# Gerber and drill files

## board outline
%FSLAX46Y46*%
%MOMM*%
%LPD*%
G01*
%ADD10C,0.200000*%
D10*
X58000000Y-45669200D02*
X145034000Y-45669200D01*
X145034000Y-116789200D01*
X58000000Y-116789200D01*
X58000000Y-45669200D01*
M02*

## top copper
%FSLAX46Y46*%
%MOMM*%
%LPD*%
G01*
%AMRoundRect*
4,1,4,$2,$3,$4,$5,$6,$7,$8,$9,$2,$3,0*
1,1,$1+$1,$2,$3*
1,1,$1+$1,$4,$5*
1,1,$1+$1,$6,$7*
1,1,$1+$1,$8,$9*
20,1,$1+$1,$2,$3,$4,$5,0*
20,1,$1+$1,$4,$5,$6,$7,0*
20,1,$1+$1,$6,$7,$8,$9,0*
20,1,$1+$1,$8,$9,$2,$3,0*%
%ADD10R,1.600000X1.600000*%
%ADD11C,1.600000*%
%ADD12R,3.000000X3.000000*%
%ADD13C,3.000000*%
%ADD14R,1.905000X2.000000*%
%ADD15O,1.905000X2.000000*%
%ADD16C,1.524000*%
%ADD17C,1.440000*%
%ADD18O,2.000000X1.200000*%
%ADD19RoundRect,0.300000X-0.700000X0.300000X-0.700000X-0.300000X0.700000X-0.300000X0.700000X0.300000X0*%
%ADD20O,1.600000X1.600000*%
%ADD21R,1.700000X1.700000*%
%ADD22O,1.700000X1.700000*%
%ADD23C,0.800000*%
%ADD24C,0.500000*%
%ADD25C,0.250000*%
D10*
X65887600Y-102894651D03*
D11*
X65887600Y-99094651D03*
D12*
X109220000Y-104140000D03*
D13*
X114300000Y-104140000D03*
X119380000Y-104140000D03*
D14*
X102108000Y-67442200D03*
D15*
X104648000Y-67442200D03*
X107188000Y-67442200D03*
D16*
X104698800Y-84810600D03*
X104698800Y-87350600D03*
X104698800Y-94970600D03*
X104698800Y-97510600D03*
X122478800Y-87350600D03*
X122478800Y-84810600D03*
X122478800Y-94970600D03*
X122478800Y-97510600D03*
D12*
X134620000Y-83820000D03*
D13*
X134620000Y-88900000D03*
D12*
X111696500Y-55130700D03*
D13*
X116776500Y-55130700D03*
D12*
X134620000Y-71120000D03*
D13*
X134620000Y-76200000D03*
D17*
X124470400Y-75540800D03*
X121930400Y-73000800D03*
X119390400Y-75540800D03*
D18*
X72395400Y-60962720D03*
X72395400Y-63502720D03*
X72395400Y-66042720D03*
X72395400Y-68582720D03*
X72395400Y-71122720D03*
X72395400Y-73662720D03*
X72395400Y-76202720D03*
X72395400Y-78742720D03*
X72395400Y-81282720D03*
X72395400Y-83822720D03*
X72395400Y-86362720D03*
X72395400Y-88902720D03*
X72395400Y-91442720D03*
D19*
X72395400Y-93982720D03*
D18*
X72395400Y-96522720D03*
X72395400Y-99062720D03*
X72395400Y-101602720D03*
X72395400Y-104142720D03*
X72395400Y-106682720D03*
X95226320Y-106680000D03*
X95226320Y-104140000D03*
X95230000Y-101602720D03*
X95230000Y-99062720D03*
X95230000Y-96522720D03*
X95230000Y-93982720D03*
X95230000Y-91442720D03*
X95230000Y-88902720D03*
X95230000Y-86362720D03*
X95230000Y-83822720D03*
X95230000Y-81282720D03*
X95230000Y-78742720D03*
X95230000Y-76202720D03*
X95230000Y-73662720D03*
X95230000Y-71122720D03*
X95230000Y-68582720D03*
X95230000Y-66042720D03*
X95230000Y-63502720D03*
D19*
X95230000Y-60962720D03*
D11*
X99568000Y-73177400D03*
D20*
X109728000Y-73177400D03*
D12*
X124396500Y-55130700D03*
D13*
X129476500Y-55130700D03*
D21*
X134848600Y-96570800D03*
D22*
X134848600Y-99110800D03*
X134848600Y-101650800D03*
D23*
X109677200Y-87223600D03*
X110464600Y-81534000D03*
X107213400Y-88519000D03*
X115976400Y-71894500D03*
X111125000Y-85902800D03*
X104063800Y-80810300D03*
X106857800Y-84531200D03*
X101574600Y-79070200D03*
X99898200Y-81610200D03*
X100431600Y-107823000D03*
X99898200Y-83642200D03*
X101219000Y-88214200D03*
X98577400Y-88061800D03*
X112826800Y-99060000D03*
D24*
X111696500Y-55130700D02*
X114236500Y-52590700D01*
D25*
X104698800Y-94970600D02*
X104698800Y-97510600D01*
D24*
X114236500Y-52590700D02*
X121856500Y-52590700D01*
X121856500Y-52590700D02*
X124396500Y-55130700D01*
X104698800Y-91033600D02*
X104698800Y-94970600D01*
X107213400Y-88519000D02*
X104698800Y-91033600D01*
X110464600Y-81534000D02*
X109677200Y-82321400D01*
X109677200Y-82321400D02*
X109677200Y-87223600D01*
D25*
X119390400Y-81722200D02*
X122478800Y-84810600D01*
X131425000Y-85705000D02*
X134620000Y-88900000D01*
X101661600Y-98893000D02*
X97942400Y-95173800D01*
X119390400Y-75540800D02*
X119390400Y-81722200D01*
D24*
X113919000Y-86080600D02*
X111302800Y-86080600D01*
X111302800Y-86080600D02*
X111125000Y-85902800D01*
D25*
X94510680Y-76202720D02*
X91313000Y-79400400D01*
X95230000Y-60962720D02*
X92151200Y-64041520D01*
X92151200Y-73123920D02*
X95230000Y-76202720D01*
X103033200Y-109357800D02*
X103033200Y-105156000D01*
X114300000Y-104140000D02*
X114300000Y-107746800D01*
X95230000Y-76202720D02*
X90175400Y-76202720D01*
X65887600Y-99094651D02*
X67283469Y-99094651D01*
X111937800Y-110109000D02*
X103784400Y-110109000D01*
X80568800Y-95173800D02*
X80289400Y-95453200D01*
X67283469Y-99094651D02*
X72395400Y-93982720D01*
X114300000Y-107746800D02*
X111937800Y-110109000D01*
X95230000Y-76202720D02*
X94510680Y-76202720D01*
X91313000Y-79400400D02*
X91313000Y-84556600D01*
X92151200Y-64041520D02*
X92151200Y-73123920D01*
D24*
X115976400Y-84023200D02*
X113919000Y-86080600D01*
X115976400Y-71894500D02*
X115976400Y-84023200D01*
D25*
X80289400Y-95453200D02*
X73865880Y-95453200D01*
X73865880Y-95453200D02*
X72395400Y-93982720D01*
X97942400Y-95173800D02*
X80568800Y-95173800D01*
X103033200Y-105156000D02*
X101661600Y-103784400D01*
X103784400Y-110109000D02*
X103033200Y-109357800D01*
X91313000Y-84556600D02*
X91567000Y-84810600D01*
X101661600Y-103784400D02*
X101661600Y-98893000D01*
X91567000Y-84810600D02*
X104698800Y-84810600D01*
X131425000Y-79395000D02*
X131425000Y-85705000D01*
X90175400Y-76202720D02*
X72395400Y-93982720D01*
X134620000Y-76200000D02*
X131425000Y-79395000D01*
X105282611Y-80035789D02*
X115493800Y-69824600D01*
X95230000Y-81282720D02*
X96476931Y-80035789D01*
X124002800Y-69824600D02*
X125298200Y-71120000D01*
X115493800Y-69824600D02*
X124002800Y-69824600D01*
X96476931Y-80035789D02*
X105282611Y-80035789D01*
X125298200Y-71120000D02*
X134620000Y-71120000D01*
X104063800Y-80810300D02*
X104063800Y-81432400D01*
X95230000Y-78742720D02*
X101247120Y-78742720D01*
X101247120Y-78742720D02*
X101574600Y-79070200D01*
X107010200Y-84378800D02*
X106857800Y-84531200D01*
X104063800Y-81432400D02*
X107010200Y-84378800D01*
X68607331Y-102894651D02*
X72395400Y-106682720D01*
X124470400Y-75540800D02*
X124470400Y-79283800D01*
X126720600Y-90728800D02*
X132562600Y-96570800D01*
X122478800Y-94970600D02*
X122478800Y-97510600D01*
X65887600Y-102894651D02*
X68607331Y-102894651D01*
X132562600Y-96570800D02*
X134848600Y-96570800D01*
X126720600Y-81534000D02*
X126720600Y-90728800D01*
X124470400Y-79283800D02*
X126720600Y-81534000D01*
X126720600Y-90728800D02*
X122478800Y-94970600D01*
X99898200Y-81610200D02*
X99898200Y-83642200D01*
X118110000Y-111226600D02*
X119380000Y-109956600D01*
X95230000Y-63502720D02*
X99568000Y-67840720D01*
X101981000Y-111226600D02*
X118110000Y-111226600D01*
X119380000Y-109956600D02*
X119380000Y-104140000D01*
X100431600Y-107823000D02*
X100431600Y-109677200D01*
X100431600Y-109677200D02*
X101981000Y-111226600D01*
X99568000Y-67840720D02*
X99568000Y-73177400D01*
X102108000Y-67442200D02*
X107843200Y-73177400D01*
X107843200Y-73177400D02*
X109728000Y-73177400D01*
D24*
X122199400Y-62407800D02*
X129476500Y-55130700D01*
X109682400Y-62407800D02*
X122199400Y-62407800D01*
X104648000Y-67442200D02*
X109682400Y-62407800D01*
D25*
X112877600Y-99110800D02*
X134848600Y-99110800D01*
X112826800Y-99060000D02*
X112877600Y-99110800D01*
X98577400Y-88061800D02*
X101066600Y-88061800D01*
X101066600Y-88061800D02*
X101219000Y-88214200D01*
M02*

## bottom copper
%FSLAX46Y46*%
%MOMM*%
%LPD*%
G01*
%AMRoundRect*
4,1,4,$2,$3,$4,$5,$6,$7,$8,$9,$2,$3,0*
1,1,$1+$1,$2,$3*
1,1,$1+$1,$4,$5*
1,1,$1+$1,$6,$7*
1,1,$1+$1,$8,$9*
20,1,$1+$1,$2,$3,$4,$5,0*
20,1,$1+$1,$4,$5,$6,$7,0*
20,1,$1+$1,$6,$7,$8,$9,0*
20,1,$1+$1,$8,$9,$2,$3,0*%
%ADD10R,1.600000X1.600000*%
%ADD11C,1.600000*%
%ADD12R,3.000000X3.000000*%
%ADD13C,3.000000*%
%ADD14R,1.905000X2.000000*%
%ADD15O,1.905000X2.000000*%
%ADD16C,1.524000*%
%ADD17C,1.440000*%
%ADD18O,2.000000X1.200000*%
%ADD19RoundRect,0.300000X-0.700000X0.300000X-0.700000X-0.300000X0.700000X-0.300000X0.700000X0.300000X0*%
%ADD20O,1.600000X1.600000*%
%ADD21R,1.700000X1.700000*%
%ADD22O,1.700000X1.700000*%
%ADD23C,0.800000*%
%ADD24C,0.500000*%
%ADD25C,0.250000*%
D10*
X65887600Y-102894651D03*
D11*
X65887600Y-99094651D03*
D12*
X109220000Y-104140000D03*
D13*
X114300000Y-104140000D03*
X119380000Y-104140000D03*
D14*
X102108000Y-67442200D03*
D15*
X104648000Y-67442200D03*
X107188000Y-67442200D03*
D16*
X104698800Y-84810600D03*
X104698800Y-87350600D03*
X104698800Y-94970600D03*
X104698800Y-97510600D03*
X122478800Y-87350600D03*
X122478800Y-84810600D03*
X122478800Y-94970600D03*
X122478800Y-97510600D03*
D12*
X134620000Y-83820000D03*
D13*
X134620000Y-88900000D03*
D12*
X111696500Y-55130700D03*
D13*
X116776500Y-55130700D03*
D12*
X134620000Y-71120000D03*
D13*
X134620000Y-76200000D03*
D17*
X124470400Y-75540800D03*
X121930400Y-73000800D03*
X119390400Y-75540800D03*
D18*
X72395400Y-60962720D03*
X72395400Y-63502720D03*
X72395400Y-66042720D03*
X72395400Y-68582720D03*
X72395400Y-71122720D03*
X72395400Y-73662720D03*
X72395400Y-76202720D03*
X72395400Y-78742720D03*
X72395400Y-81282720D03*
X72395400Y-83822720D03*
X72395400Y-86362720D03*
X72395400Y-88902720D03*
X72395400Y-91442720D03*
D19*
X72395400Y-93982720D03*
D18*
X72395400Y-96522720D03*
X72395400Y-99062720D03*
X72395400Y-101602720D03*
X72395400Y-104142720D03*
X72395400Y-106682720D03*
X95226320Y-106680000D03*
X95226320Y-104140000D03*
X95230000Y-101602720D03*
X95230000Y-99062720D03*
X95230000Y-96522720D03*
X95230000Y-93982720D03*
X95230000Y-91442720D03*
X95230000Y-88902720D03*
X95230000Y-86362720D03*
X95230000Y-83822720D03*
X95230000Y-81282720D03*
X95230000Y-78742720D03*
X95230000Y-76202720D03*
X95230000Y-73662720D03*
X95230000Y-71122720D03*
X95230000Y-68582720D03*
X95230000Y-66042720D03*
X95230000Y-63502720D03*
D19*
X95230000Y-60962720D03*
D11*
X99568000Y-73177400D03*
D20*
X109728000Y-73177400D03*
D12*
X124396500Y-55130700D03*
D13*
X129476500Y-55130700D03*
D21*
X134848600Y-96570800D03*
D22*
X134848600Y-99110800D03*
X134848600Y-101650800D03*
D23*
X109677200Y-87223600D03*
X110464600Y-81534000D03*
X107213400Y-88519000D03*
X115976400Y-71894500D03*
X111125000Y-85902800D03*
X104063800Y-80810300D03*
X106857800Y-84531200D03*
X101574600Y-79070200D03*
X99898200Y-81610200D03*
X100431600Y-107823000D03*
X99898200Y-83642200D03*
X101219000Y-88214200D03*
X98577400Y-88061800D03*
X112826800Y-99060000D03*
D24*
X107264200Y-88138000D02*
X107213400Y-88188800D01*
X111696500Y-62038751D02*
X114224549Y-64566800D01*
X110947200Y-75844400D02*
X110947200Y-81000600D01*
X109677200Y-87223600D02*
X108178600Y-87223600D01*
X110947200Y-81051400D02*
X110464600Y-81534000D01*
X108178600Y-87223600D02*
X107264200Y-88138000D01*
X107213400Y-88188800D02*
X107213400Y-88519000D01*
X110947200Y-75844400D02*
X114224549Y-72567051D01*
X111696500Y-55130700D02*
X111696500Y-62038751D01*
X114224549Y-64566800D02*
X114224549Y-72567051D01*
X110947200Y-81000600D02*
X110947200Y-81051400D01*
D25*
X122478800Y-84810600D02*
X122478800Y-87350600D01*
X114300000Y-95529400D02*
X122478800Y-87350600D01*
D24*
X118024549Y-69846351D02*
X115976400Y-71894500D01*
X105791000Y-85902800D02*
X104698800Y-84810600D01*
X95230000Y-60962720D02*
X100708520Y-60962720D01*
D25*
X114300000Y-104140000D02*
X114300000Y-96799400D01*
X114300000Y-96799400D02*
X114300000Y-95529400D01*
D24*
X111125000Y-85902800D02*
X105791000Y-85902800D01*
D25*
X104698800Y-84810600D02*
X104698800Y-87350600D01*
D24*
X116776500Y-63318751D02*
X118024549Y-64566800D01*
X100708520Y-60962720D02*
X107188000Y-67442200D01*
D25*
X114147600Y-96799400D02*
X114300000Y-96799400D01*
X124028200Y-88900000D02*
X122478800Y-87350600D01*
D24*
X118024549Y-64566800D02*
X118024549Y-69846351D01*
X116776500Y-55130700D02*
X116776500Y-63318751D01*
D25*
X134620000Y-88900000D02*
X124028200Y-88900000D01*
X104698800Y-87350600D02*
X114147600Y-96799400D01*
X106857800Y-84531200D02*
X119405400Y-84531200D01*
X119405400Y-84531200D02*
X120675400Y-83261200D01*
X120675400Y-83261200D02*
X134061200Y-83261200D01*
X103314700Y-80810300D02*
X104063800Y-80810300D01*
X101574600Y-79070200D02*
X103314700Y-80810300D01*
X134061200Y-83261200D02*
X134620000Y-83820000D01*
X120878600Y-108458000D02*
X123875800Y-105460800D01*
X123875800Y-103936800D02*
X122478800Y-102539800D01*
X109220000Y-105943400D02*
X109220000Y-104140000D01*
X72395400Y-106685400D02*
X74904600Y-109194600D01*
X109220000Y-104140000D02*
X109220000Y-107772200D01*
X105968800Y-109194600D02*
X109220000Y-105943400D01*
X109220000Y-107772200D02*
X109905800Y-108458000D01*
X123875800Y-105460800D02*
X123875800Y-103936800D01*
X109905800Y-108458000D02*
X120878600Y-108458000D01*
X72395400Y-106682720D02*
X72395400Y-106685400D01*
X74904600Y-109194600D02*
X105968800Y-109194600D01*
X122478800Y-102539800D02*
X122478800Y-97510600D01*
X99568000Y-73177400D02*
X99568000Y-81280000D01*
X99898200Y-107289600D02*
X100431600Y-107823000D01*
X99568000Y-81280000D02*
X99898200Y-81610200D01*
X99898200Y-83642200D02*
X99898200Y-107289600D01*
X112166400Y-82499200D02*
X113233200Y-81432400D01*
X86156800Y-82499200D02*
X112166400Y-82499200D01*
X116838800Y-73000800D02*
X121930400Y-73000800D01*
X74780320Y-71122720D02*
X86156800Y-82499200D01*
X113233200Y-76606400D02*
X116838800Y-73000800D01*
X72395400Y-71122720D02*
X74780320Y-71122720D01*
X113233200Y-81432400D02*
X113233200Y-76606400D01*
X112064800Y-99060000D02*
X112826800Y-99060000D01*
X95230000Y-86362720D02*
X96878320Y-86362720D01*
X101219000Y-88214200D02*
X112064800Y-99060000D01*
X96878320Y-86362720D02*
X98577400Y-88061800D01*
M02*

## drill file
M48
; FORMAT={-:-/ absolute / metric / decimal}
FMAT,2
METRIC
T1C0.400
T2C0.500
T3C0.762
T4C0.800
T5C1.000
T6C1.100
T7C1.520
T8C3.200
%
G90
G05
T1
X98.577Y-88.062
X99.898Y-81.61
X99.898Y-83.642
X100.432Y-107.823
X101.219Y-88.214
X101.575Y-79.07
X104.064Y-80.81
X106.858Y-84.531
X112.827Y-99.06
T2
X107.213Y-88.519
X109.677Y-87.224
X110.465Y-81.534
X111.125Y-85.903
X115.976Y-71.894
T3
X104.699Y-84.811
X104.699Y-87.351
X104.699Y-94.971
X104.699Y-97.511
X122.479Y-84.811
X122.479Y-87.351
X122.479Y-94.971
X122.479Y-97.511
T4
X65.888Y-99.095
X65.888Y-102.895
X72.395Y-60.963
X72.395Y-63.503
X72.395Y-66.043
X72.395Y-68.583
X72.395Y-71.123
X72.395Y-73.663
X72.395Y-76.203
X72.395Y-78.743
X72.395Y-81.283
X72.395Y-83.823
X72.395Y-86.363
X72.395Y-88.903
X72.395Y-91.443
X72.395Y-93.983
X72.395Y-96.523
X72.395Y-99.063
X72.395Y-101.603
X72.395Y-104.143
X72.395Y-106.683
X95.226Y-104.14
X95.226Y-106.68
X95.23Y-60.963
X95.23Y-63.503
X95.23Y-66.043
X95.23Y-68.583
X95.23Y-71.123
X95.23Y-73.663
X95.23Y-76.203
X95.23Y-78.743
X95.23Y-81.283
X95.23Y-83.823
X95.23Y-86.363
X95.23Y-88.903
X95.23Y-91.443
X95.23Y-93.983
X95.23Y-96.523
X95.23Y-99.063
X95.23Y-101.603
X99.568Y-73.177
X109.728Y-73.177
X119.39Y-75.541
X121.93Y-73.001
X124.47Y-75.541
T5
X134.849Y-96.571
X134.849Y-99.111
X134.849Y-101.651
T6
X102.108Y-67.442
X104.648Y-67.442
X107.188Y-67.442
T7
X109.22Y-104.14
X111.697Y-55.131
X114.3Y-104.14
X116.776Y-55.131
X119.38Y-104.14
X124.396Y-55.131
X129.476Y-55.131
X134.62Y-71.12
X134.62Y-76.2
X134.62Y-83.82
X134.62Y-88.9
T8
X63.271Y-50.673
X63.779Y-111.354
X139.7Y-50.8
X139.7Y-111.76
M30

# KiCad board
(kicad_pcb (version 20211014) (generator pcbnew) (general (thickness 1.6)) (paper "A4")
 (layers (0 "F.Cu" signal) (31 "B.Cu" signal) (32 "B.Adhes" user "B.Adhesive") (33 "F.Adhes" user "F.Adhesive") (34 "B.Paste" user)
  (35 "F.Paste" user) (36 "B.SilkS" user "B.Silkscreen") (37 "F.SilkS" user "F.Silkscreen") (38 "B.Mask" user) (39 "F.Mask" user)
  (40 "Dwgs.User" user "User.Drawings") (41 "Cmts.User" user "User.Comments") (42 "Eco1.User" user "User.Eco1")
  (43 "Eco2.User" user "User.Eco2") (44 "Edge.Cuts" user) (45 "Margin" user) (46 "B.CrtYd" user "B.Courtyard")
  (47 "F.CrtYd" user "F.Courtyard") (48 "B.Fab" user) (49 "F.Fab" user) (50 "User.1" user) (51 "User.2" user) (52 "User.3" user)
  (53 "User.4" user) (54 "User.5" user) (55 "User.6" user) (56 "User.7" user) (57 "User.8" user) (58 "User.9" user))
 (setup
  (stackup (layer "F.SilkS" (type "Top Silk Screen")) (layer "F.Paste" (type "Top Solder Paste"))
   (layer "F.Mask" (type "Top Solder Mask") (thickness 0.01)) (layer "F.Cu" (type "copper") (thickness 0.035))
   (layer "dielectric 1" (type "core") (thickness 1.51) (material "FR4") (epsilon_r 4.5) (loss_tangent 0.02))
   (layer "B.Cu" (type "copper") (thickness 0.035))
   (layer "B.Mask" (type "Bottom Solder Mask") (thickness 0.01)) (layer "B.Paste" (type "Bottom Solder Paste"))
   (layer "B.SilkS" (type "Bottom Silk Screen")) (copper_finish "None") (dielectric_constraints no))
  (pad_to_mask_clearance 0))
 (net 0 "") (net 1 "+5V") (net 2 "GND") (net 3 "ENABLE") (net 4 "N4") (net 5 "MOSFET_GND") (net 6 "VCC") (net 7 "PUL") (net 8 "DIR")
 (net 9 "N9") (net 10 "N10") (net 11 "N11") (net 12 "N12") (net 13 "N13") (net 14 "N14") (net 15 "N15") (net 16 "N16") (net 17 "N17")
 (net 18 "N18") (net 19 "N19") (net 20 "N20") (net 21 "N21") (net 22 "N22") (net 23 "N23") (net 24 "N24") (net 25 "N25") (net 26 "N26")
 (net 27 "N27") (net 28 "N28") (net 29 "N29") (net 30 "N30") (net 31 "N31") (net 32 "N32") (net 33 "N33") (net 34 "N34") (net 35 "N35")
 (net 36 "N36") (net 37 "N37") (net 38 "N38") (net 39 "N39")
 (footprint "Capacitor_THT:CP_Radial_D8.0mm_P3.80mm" (layer "F.Cu") (at 65.8876 102.894651 90)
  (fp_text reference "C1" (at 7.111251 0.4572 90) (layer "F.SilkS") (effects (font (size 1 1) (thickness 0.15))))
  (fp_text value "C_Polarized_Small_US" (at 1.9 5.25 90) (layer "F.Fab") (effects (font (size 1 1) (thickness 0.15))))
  (pad "1" thru_hole rect (at 0 0 90) (size 1.6 1.6) (drill 0.8) (layers *.Cu *.Mask) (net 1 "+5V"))
  (pad "2" thru_hole circle (at 3.8 0 90) (size 1.6 1.6) (drill 0.8) (layers *.Cu *.Mask) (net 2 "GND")))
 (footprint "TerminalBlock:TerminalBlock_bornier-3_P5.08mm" (layer "F.Cu") (at 109.22 104.14)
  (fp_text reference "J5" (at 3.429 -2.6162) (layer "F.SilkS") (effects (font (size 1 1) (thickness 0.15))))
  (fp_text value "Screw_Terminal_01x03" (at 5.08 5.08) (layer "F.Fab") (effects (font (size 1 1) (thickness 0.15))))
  (pad "1" thru_hole rect (at 0 0) (size 3 3) (drill 1.52) (layers *.Cu *.Mask) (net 1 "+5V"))
  (pad "2" thru_hole circle (at 5.08 0) (size 3 3) (drill 1.52) (layers *.Cu *.Mask) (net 2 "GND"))
  (pad "3" thru_hole circle (at 10.16 0) (size 3 3) (drill 1.52) (layers *.Cu *.Mask) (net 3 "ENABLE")))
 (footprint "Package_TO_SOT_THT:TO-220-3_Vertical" (layer "F.Cu") (at 102.108 67.4422)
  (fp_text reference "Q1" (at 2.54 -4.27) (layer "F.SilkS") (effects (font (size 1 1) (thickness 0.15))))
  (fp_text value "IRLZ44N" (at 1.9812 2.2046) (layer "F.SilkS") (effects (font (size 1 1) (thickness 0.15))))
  (pad "1" thru_hole rect (at 0 0) (size 1.905 2) (drill 1.1) (layers *.Cu *.Mask) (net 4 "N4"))
  (pad "2" thru_hole oval (at 2.54 0) (size 1.905 2) (drill 1.1) (layers *.Cu *.Mask) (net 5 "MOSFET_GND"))
  (pad "3" thru_hole oval (at 5.08 0) (size 1.905 2) (drill 1.1) (layers *.Cu *.Mask) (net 2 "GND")))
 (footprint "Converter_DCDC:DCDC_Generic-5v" (layer "F.Cu") (at 114.8588 92.4306)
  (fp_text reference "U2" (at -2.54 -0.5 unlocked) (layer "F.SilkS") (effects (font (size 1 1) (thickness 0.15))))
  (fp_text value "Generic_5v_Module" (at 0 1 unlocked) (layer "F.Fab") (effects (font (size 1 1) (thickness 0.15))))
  (pad "1" thru_hole circle (at -10.16 -7.62) (size 1.524 1.524) (drill 0.762) (layers *.Cu *.Mask) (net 2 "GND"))
  (pad "1" thru_hole circle (at -10.16 -5.08) (size 1.524 1.524) (drill 0.762) (layers *.Cu *.Mask) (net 2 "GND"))
  (pad "2" thru_hole circle (at -10.16 2.54) (size 1.524 1.524) (drill 0.762) (layers *.Cu *.Mask) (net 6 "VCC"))
  (pad "2" thru_hole circle (at -10.16 5.08) (size 1.524 1.524) (drill 0.762) (layers *.Cu *.Mask) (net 6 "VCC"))
  (pad "3" thru_hole circle (at 7.62 -5.08) (size 1.524 1.524) (drill 0.762) (layers *.Cu *.Mask) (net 2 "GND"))
  (pad "3" thru_hole circle (at 7.62 -7.62) (size 1.524 1.524) (drill 0.762) (layers *.Cu *.Mask) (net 2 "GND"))
  (pad "4" thru_hole circle (at 7.62 2.54) (size 1.524 1.524) (drill 0.762) (layers *.Cu *.Mask) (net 1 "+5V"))
  (pad "4" thru_hole circle (at 7.62 5.08) (size 1.524 1.524) (drill 0.762) (layers *.Cu *.Mask) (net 1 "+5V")))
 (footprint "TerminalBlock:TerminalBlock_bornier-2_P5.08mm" (layer "F.Cu") (at 134.62 83.82 -90)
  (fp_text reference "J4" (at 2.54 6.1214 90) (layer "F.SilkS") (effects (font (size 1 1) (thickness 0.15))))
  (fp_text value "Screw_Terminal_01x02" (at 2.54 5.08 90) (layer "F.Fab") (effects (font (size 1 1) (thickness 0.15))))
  (pad "1" thru_hole rect (at 0 0 270) (size 3 3) (drill 1.52) (layers *.Cu *.Mask) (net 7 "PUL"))
  (pad "2" thru_hole circle (at 5.08 0 270) (size 3 3) (drill 1.52) (layers *.Cu *.Mask) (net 2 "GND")))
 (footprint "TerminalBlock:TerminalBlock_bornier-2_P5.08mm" (layer "F.Cu") (at 111.6965 55.1307)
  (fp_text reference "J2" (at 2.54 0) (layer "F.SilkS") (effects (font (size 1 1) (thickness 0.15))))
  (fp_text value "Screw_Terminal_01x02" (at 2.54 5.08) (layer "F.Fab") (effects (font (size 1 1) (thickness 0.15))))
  (pad "1" thru_hole rect (at 0 0) (size 3 3) (drill 1.52) (layers *.Cu *.Mask) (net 6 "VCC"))
  (pad "2" thru_hole circle (at 5.08 0) (size 3 3) (drill 1.52) (layers *.Cu *.Mask) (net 2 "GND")))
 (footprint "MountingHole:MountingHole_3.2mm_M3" (layer "F.Cu") (at 63.2714 50.673)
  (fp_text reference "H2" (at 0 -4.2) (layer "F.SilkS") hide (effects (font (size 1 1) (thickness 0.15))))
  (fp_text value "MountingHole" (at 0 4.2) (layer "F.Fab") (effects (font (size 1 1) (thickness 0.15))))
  (pad "" np_thru_hole circle (at 0 0) (size 3.2 3.2) (drill 3.2) (layers *.Cu *.Mask)))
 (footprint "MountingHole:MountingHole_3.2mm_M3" (layer "F.Cu") (at 139.7 111.76)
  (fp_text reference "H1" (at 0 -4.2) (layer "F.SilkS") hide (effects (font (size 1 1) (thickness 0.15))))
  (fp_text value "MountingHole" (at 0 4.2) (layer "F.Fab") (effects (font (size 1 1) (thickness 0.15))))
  (pad "" np_thru_hole circle (at 0 0) (size 3.2 3.2) (drill 3.2) (layers *.Cu *.Mask)))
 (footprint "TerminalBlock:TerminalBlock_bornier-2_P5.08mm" (layer "F.Cu") (at 134.62 71.12 -90)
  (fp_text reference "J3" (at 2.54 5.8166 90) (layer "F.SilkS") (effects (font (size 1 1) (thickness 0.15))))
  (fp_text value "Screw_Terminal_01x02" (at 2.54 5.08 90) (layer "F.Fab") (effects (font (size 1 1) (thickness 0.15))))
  (pad "1" thru_hole rect (at 0 0 270) (size 3 3) (drill 1.52) (layers *.Cu *.Mask) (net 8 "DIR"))
  (pad "2" thru_hole circle (at 5.08 0 270) (size 3 3) (drill 1.52) (layers *.Cu *.Mask) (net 2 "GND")))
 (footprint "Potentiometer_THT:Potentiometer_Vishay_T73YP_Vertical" (layer "F.Cu") (at 124.4704 75.5408 90)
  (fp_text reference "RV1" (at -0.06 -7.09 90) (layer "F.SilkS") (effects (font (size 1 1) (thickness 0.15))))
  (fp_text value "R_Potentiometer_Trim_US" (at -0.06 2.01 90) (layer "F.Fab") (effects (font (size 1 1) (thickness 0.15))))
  (pad "1" thru_hole circle (at 0 0 90) (size 1.44 1.44) (drill 0.8) (layers *.Cu *.Mask) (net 1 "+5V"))
  (pad "2" thru_hole circle (at 2.54 -2.54 90) (size 1.44 1.44) (drill 0.8) (layers *.Cu *.Mask) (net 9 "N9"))
  (pad "3" thru_hole circle (at 0 -5.08 90) (size 1.44 1.44) (drill 0.8) (layers *.Cu *.Mask) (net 2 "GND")))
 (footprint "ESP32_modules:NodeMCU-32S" (layer "F.Cu") (at 71.12 60.96)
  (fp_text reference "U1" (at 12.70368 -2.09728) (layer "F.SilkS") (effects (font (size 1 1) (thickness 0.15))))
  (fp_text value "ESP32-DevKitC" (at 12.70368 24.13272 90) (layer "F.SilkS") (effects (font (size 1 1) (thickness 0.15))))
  (pad "1" thru_hole oval (at 1.2754 0.00272 270) (size 1.2 2) (drill 0.8) (layers *.Cu *.Mask) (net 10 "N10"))
  (pad "2" thru_hole oval (at 1.2754 2.54272 270) (size 1.2 2) (drill 0.8) (layers *.Cu *.Mask) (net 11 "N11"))
  (pad "3" thru_hole oval (at 1.2754 5.08272 270) (size 1.2 2) (drill 0.8) (layers *.Cu *.Mask) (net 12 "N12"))
  (pad "4" thru_hole oval (at 1.2754 7.62272 270) (size 1.2 2) (drill 0.8) (layers *.Cu *.Mask) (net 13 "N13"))
  (pad "5" thru_hole oval (at 1.2754 10.16272 270) (size 1.2 2) (drill 0.8) (layers *.Cu *.Mask) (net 9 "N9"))
  (pad "6" thru_hole oval (at 1.2754 12.70272 270) (size 1.2 2) (drill 0.8) (layers *.Cu *.Mask) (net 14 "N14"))
  (pad "7" thru_hole oval (at 1.2754 15.24272 270) (size 1.2 2) (drill 0.8) (layers *.Cu *.Mask) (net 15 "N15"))
  (pad "8" thru_hole oval (at 1.2754 17.78272 270) (size 1.2 2) (drill 0.8) (layers *.Cu *.Mask) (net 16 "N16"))
  (pad "9" thru_hole oval (at 1.2754 20.32272 270) (size 1.2 2) (drill 0.8) (layers *.Cu *.Mask) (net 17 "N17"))
  (pad "10" thru_hole oval (at 1.2754 22.86272 270) (size 1.2 2) (drill 0.8) (layers *.Cu *.Mask) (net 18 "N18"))
  (pad "11" thru_hole oval (at 1.2754 25.40272 270) (size 1.2 2) (drill 0.8) (layers *.Cu *.Mask) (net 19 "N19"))
  (pad "12" thru_hole oval (at 1.2754 27.94272 270) (size 1.2 2) (drill 0.8) (layers *.Cu *.Mask) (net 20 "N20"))
  (pad "13" thru_hole oval (at 1.2754 30.48272 270) (size 1.2 2) (drill 0.8) (layers *.Cu *.Mask) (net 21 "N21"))
  (pad "14" thru_hole roundrect (at 1.2754 33.02272 270) (size 1.2 2) (drill 0.8) (layers *.Cu *.Mask) (roundrect_rratio 0.25) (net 2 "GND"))
  (pad "15" thru_hole oval (at 1.2754 35.56272 270) (size 1.2 2) (drill 0.8) (layers *.Cu *.Mask) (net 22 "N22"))
  (pad "16" thru_hole oval (at 1.2754 38.10272 270) (size 1.2 2) (drill 0.8) (layers *.Cu *.Mask) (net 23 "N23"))
  (pad "17" thru_hole oval (at 1.2754 40.64272 270) (size 1.2 2) (drill 0.8) (layers *.Cu *.Mask) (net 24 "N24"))
  (pad "18" thru_hole oval (at 1.2754 43.18272 270) (size 1.2 2) (drill 0.8) (layers *.Cu *.Mask) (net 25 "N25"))
  (pad "19" thru_hole oval (at 1.2754 45.72272 270) (size 1.2 2) (drill 0.8) (layers *.Cu *.Mask) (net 1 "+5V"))
  (pad "20" thru_hole oval (at 24.10632 45.72 270) (size 1.2 2) (drill 0.8) (layers *.Cu *.Mask) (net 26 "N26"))
  (pad "21" thru_hole oval (at 24.10632 43.18 270) (size 1.2 2) (drill 0.8) (layers *.Cu *.Mask) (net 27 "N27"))
  (pad "22" thru_hole oval (at 24.11 40.64272 270) (size 1.2 2) (drill 0.8) (layers *.Cu *.Mask) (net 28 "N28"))
  (pad "23" thru_hole oval (at 24.11 38.10272 270) (size 1.2 2) (drill 0.8) (layers *.Cu *.Mask) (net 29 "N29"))
  (pad "24" thru_hole oval (at 24.11 35.56272 270) (size 1.2 2) (drill 0.8) (layers *.Cu *.Mask) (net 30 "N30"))
  (pad "25" thru_hole oval (at 24.11 33.02272 270) (size 1.2 2) (drill 0.8) (layers *.Cu *.Mask) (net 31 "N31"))
  (pad "26" thru_hole oval (at 24.11 30.48272 270) (size 1.2 2) (drill 0.8) (layers *.Cu *.Mask) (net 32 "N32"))
  (pad "27" thru_hole oval (at 24.11 27.94272 270) (size 1.2 2) (drill 0.8) (layers *.Cu *.Mask) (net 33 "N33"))
  (pad "28" thru_hole oval (at 24.11 25.40272 270) (size 1.2 2) (drill 0.8) (layers *.Cu *.Mask) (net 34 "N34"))
  (pad "29" thru_hole oval (at 24.11 22.86272 270) (size 1.2 2) (drill 0.8) (layers *.Cu *.Mask) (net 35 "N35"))
  (pad "30" thru_hole oval (at 24.11 20.32272 270) (size 1.2 2) (drill 0.8) (layers *.Cu *.Mask) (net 8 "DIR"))
  (pad "31" thru_hole oval (at 24.11 17.78272 270) (size 1.2 2) (drill 0.8) (layers *.Cu *.Mask) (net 7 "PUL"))
  (pad "32" thru_hole oval (at 24.11 15.24272 270) (size 1.2 2) (drill 0.8) (layers *.Cu *.Mask) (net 2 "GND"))
  (pad "33" thru_hole oval (at 24.11 12.70272 270) (size 1.2 2) (drill 0.8) (layers *.Cu *.Mask) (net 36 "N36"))
  (pad "34" thru_hole oval (at 24.11 10.16272 270) (size 1.2 2) (drill 0.8) (layers *.Cu *.Mask) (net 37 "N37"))
  (pad "35" thru_hole oval (at 24.11 7.62272 270) (size 1.2 2) (drill 0.8) (layers *.Cu *.Mask) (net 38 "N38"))
  (pad "36" thru_hole oval (at 24.11 5.08272 270) (size 1.2 2) (drill 0.8) (layers *.Cu *.Mask) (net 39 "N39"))
  (pad "37" thru_hole oval (at 24.11 2.54272 270) (size 1.2 2) (drill 0.8) (layers *.Cu *.Mask) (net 3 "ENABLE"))
  (pad "38" thru_hole roundrect (at 24.11 0.00272 270) (size 1.2 2) (drill 0.8) (layers *.Cu *.Mask) (roundrect_rratio 0.25) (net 2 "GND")))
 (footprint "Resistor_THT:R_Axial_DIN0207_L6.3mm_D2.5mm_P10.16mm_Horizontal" (layer "F.Cu") (at 99.568 73.1774)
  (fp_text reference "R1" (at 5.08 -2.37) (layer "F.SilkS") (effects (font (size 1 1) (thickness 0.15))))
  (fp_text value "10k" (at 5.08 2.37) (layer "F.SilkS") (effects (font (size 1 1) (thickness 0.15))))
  (pad "1" thru_hole circle (at 0 0) (size 1.6 1.6) (drill 0.8) (layers *.Cu *.Mask) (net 3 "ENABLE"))
  (pad "2" thru_hole oval (at 10.16 0) (size 1.6 1.6) (drill 0.8) (layers *.Cu *.Mask) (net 4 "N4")))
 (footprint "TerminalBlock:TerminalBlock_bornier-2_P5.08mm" (layer "F.Cu") (at 124.3965 55.1307)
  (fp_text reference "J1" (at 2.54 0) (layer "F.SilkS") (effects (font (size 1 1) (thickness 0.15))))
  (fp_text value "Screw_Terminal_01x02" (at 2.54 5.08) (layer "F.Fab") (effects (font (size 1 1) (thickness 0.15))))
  (pad "1" thru_hole rect (at 0 0) (size 3 3) (drill 1.52) (layers *.Cu *.Mask) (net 6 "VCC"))
  (pad "2" thru_hole circle (at 5.08 0) (size 3 3) (drill 1.52) (layers *.Cu *.Mask) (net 5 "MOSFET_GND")))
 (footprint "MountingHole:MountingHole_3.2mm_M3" (layer "F.Cu") (at 63.7794 111.3536)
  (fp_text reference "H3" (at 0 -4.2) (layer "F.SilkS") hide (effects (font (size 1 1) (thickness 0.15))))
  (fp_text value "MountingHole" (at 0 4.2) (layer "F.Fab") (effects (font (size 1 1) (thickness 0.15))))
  (pad "" np_thru_hole circle (at 0 0) (size 3.2 3.2) (drill 3.2) (layers *.Cu *.Mask)))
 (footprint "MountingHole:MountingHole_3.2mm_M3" (layer "F.Cu") (at 139.7 50.8)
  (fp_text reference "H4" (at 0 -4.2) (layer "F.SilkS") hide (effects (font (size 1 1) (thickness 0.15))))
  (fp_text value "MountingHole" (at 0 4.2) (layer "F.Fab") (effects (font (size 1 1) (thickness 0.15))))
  (pad "" np_thru_hole circle (at 0 0) (size 3.2 3.2) (drill 3.2) (layers F&B.Cu *.Mask)))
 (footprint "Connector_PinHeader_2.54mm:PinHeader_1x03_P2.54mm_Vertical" (layer "F.Cu") (at 134.8486 96.5708)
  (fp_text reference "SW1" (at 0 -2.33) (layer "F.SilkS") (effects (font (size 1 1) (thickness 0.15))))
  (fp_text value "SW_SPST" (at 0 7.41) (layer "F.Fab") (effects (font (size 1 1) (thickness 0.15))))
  (pad "1" thru_hole rect (at 0 0) (size 1.7 1.7) (drill 1) (layers *.Cu *.Mask) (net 1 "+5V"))
  (pad "2" thru_hole oval (at 0 2.54) (size 1.7 1.7) (drill 1) (layers *.Cu *.Mask) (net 34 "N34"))
  (pad "3" thru_hole oval (at 0 5.08) (size 1.7 1.7) (drill 1) (layers *.Cu *.Mask)))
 (gr_rect (start 58 45.6692) (end 145.034 116.7892) (layer "Edge.Cuts") (width 0.2) (fill none))
 (segment (start 111.6965 55.1307) (end 114.2365 52.5907) (width 0.5) (layer "F.Cu") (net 6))
 (segment (start 104.6988 94.9706) (end 104.6988 97.5106) (width 0.25) (layer "F.Cu") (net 6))
 (segment (start 114.2365 52.5907) (end 121.8565 52.5907) (width 0.5) (layer "F.Cu") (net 6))
 (segment (start 121.8565 52.5907) (end 124.3965 55.1307) (width 0.5) (layer "F.Cu") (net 6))
 (segment (start 104.6988 91.0336) (end 104.6988 94.9706) (width 0.5) (layer "F.Cu") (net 6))
 (segment (start 107.2134 88.519) (end 104.6988 91.0336) (width 0.5) (layer "F.Cu") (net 6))
 (segment (start 110.4646 81.534) (end 109.6772 82.3214) (width 0.5) (layer "F.Cu") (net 6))
 (segment (start 109.6772 82.3214) (end 109.6772 87.2236) (width 0.5) (layer "F.Cu") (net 6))
 (via (at 109.6772 87.2236) (size 0.8) (drill 0.5) (layers "F.Cu" "B.Cu") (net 6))
 (via (at 110.4646 81.534) (size 0.8) (drill 0.5) (layers "F.Cu" "B.Cu") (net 6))
 (via (at 107.2134 88.519) (size 0.8) (drill 0.5) (layers "F.Cu" "B.Cu") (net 6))
 (segment (start 107.2642 88.138) (end 107.2134 88.1888) (width 0.5) (layer "B.Cu") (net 6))
 (segment (start 111.6965 62.038751) (end 114.224549 64.5668) (width 0.5) (layer "B.Cu") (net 6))
 (segment (start 110.9472 75.8444) (end 110.9472 81.0006) (width 0.5) (layer "B.Cu") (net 6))
 (segment (start 109.6772 87.2236) (end 108.1786 87.2236) (width 0.5) (layer "B.Cu") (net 6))
 (segment (start 110.9472 81.0514) (end 110.4646 81.534) (width 0.5) (layer "B.Cu") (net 6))
 (segment (start 108.1786 87.2236) (end 107.2642 88.138) (width 0.5) (layer "B.Cu") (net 6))
 (segment (start 107.2134 88.1888) (end 107.2134 88.519) (width 0.5) (layer "B.Cu") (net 6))
 (segment (start 110.9472 75.8444) (end 114.224549 72.567051) (width 0.5) (layer "B.Cu") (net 6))
 (segment (start 111.6965 55.1307) (end 111.6965 62.038751) (width 0.5) (layer "B.Cu") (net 6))
 (segment (start 114.224549 64.5668) (end 114.224549 72.567051) (width 0.5) (layer "B.Cu") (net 6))
 (segment (start 110.9472 81.0006) (end 110.9472 81.0514) (width 0.5) (layer "B.Cu") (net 6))
 (segment (start 119.3904 81.7222) (end 122.4788 84.8106) (width 0.25) (layer "F.Cu") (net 2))
 (segment (start 131.425 85.705) (end 134.62 88.9) (width 0.25) (layer "F.Cu") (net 2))
 (segment (start 101.6616 98.893) (end 97.9424 95.1738) (width 0.25) (layer "F.Cu") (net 2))
 (segment (start 119.3904 75.5408) (end 119.3904 81.7222) (width 0.25) (layer "F.Cu") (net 2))
 (segment (start 113.919 86.0806) (end 111.3028 86.0806) (width 0.5) (layer "F.Cu") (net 2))
 (segment (start 111.3028 86.0806) (end 111.125 85.9028) (width 0.5) (layer "F.Cu") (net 2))
 (segment (start 94.51068 76.20272) (end 91.313 79.4004) (width 0.25) (layer "F.Cu") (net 2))
 (segment (start 95.23 60.96272) (end 92.1512 64.04152) (width 0.25) (layer "F.Cu") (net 2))
 (segment (start 92.1512 73.12392) (end 95.23 76.20272) (width 0.25) (layer "F.Cu") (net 2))
 (segment (start 103.0332 109.3578) (end 103.0332 105.156) (width 0.25) (layer "F.Cu") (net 2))
 (segment (start 114.3 104.14) (end 114.3 107.7468) (width 0.25) (layer "F.Cu") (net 2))
 (segment (start 95.23 76.20272) (end 90.1754 76.20272) (width 0.25) (layer "F.Cu") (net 2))
 (segment (start 65.8876 99.094651) (end 67.283469 99.094651) (width 0.25) (layer "F.Cu") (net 2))
 (segment (start 111.9378 110.109) (end 103.7844 110.109) (width 0.25) (layer "F.Cu") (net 2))
 (segment (start 80.5688 95.1738) (end 80.2894 95.4532) (width 0.25) (layer "F.Cu") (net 2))
 (segment (start 67.283469 99.094651) (end 72.3954 93.98272) (width 0.25) (layer "F.Cu") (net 2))
 (segment (start 114.3 107.7468) (end 111.9378 110.109) (width 0.25) (layer "F.Cu") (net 2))
 (segment (start 95.23 76.20272) (end 94.51068 76.20272) (width 0.25) (layer "F.Cu") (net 2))
 (segment (start 91.313 79.4004) (end 91.313 84.5566) (width 0.25) (layer "F.Cu") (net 2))
 (segment (start 92.1512 64.04152) (end 92.1512 73.12392) (width 0.25) (layer "F.Cu") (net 2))
 (segment (start 115.9764 84.0232) (end 113.919 86.0806) (width 0.5) (layer "F.Cu") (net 2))
 (segment (start 115.9764 71.8945) (end 115.9764 84.0232) (width 0.5) (layer "F.Cu") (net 2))
 (segment (start 80.2894 95.4532) (end 73.86588 95.4532) (width 0.25) (layer "F.Cu") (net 2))
 (segment (start 73.86588 95.4532) (end 72.3954 93.98272) (width 0.25) (layer "F.Cu") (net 2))
 (segment (start 97.9424 95.1738) (end 80.5688 95.1738) (width 0.25) (layer "F.Cu") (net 2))
 (segment (start 103.0332 105.156) (end 101.6616 103.7844) (width 0.25) (layer "F.Cu") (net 2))
 (segment (start 103.7844 110.109) (end 103.0332 109.3578) (width 0.25) (layer "F.Cu") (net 2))
 (segment (start 91.313 84.5566) (end 91.567 84.8106) (width 0.25) (layer "F.Cu") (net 2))
 (segment (start 101.6616 103.7844) (end 101.6616 98.893) (width 0.25) (layer "F.Cu") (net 2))
 (segment (start 91.567 84.8106) (end 104.6988 84.8106) (width 0.25) (layer "F.Cu") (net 2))
 (segment (start 131.425 79.395) (end 131.425 85.705) (width 0.25) (layer "F.Cu") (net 2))
 (segment (start 90.1754 76.20272) (end 72.3954 93.98272) (width 0.25) (layer "F.Cu") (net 2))
 (segment (start 134.62 76.2) (end 131.425 79.395) (width 0.25) (layer "F.Cu") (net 2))
 (via (at 115.9764 71.8945) (size 0.8) (drill 0.5) (layers "F.Cu" "B.Cu") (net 2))
 (via (at 111.125 85.9028) (size 0.8) (drill 0.5) (layers "F.Cu" "B.Cu") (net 2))
 (segment (start 122.4788 84.8106) (end 122.4788 87.3506) (width 0.25) (layer "B.Cu") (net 2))
 (segment (start 114.3 95.5294) (end 122.4788 87.3506) (width 0.25) (layer "B.Cu") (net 2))
 (segment (start 118.024549 69.846351) (end 115.9764 71.8945) (width 0.5) (layer "B.Cu") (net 2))
 (segment (start 105.791 85.9028) (end 104.6988 84.8106) (width 0.5) (layer "B.Cu") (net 2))
 (segment (start 95.23 60.96272) (end 100.70852 60.96272) (width 0.5) (layer "B.Cu") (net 2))
 (segment (start 114.3 104.14) (end 114.3 96.7994) (width 0.25) (layer "B.Cu") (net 2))
 (segment (start 114.3 96.7994) (end 114.3 95.5294) (width 0.25) (layer "B.Cu") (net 2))
 (segment (start 111.125 85.9028) (end 105.791 85.9028) (width 0.5) (layer "B.Cu") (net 2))
 (segment (start 104.6988 84.8106) (end 104.6988 87.3506) (width 0.25) (layer "B.Cu") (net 2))
 (segment (start 116.7765 63.318751) (end 118.024549 64.5668) (width 0.5) (layer "B.Cu") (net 2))
 (segment (start 100.70852 60.96272) (end 107.188 67.4422) (width 0.5) (layer "B.Cu") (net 2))
 (segment (start 114.1476 96.7994) (end 114.3 96.7994) (width 0.25) (layer "B.Cu") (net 2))
 (segment (start 124.0282 88.9) (end 122.4788 87.3506) (width 0.25) (layer "B.Cu") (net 2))
 (segment (start 118.024549 64.5668) (end 118.024549 69.846351) (width 0.5) (layer "B.Cu") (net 2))
 (segment (start 116.7765 55.1307) (end 116.7765 63.318751) (width 0.5) (layer "B.Cu") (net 2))
 (segment (start 134.62 88.9) (end 124.0282 88.9) (width 0.25) (layer "B.Cu") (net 2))
 (segment (start 104.6988 87.3506) (end 114.1476 96.7994) (width 0.25) (layer "B.Cu") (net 2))
 (segment (start 105.282611 80.035789) (end 115.4938 69.8246) (width 0.25) (layer "F.Cu") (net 8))
 (segment (start 95.23 81.28272) (end 96.476931 80.035789) (width 0.25) (layer "F.Cu") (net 8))
 (segment (start 124.0028 69.8246) (end 125.2982 71.12) (width 0.25) (layer "F.Cu") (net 8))
 (segment (start 115.4938 69.8246) (end 124.0028 69.8246) (width 0.25) (layer "F.Cu") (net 8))
 (segment (start 96.476931 80.035789) (end 105.282611 80.035789) (width 0.25) (layer "F.Cu") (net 8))
 (segment (start 125.2982 71.12) (end 134.62 71.12) (width 0.25) (layer "F.Cu") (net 8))
 (segment (start 104.0638 80.8103) (end 104.0638 81.4324) (width 0.25) (layer "F.Cu") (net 7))
 (segment (start 95.23 78.74272) (end 101.24712 78.74272) (width 0.25) (layer "F.Cu") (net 7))
 (segment (start 101.24712 78.74272) (end 101.5746 79.0702) (width 0.25) (layer "F.Cu") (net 7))
 (segment (start 107.0102 84.3788) (end 106.8578 84.5312) (width 0.25) (layer "F.Cu") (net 7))
 (segment (start 104.0638 81.4324) (end 107.0102 84.3788) (width 0.25) (layer "F.Cu") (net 7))
 (via (at 104.0638 80.8103) (size 0.8) (drill 0.4) (layers "F.Cu" "B.Cu") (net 7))
 (via (at 106.8578 84.5312) (size 0.8) (drill 0.4) (layers "F.Cu" "B.Cu") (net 7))
 (via (at 101.5746 79.0702) (size 0.8) (drill 0.4) (layers "F.Cu" "B.Cu") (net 7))
 (segment (start 106.8578 84.5312) (end 119.4054 84.5312) (width 0.25) (layer "B.Cu") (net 7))
 (segment (start 119.4054 84.5312) (end 120.6754 83.2612) (width 0.25) (layer "B.Cu") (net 7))
 (segment (start 120.6754 83.2612) (end 134.0612 83.2612) (width 0.25) (layer "B.Cu") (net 7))
 (segment (start 103.3147 80.8103) (end 104.0638 80.8103) (width 0.25) (layer "B.Cu") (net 7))
 (segment (start 101.5746 79.0702) (end 103.3147 80.8103) (width 0.25) (layer "B.Cu") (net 7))
 (segment (start 134.0612 83.2612) (end 134.62 83.82) (width 0.25) (layer "B.Cu") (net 7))
 (segment (start 68.607331 102.894651) (end 72.3954 106.68272) (width 0.25) (layer "F.Cu") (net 1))
 (segment (start 124.4704 75.5408) (end 124.4704 79.2838) (width 0.25) (layer "F.Cu") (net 1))
 (segment (start 126.7206 90.7288) (end 132.5626 96.5708) (width 0.25) (layer "F.Cu") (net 1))
 (segment (start 122.4788 94.9706) (end 122.4788 97.5106) (width 0.25) (layer "F.Cu") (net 1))
 (segment (start 65.8876 102.894651) (end 68.607331 102.894651) (width 0.25) (layer "F.Cu") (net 1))
 (segment (start 132.5626 96.5708) (end 134.8486 96.5708) (width 0.25) (layer "F.Cu") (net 1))
 (segment (start 126.7206 81.534) (end 126.7206 90.7288) (width 0.25) (layer "F.Cu") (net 1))
 (segment (start 124.4704 79.2838) (end 126.7206 81.534) (width 0.25) (layer "F.Cu") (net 1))
 (segment (start 126.7206 90.7288) (end 122.4788 94.9706) (width 0.25) (layer "F.Cu") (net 1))
 (segment (start 120.8786 108.458) (end 123.8758 105.4608) (width 0.25) (layer "B.Cu") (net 1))
 (segment (start 123.8758 103.9368) (end 122.4788 102.5398) (width 0.25) (layer "B.Cu") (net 1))
 (segment (start 109.22 105.9434) (end 109.22 104.14) (width 0.25) (layer "B.Cu") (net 1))
 (segment (start 72.3954 106.6854) (end 74.9046 109.1946) (width 0.25) (layer "B.Cu") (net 1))
 (segment (start 109.22 104.14) (end 109.22 107.7722) (width 0.25) (layer "B.Cu") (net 1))
 (segment (start 105.9688 109.1946) (end 109.22 105.9434) (width 0.25) (layer "B.Cu") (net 1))
 (segment (start 109.22 107.7722) (end 109.9058 108.458) (width 0.25) (layer "B.Cu") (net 1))
 (segment (start 123.8758 105.4608) (end 123.8758 103.9368) (width 0.25) (layer "B.Cu") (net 1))
 (segment (start 109.9058 108.458) (end 120.8786 108.458) (width 0.25) (layer "B.Cu") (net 1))
 (segment (start 72.3954 106.68272) (end 72.3954 106.6854) (width 0.25) (layer "B.Cu") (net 1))
 (segment (start 74.9046 109.1946) (end 105.9688 109.1946) (width 0.25) (layer "B.Cu") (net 1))
 (segment (start 122.4788 102.5398) (end 122.4788 97.5106) (width 0.25) (layer "B.Cu") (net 1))
 (segment (start 99.8982 81.6102) (end 99.8982 83.6422) (width 0.25) (layer "F.Cu") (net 3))
 (segment (start 118.11 111.2266) (end 119.38 109.9566) (width 0.25) (layer "F.Cu") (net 3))
 (segment (start 95.23 63.50272) (end 99.568 67.84072) (width 0.25) (layer "F.Cu") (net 3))
 (segment (start 101.981 111.2266) (end 118.11 111.2266) (width 0.25) (layer "F.Cu") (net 3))
 (segment (start 119.38 109.9566) (end 119.38 104.14) (width 0.25) (layer "F.Cu") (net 3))
 (segment (start 100.4316 107.823) (end 100.4316 109.6772) (width 0.25) (layer "F.Cu") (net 3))
 (segment (start 100.4316 109.6772) (end 101.981 111.2266) (width 0.25) (layer "F.Cu") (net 3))
 (segment (start 99.568 67.84072) (end 99.568 73.1774) (width 0.25) (layer "F.Cu") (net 3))
 (via (at 99.8982 81.6102) (size 0.8) (drill 0.4) (layers "F.Cu" "B.Cu") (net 3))
 (via (at 100.4316 107.823) (size 0.8) (drill 0.4) (layers "F.Cu" "B.Cu") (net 3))
 (via (at 99.8982 83.6422) (size 0.8) (drill 0.4) (layers "F.Cu" "B.Cu") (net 3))
 (segment (start 99.568 73.1774) (end 99.568 81.28) (width 0.25) (layer "B.Cu") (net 3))
 (segment (start 99.8982 107.2896) (end 100.4316 107.823) (width 0.25) (layer "B.Cu") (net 3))
 (segment (start 99.568 81.28) (end 99.8982 81.6102) (width 0.25) (layer "B.Cu") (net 3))
 (segment (start 99.8982 83.6422) (end 99.8982 107.2896) (width 0.25) (layer "B.Cu") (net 3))
 (segment (start 102.108 67.4422) (end 107.8432 73.1774) (width 0.25) (layer "F.Cu") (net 4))
 (segment (start 107.8432 73.1774) (end 109.728 73.1774) (width 0.25) (layer "F.Cu") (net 4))
 (segment (start 122.1994 62.4078) (end 129.4765 55.1307) (width 0.5) (layer "F.Cu") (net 5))
 (segment (start 109.6824 62.4078) (end 122.1994 62.4078) (width 0.5) (layer "F.Cu") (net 5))
 (segment (start 104.648 67.4422) (end 109.6824 62.4078) (width 0.5) (layer "F.Cu") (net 5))
 (segment (start 112.1664 82.4992) (end 113.2332 81.4324) (width 0.25) (layer "B.Cu") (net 9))
 (segment (start 86.1568 82.4992) (end 112.1664 82.4992) (width 0.25) (layer "B.Cu") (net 9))
 (segment (start 116.8388 73.0008) (end 121.9304 73.0008) (width 0.25) (layer "B.Cu") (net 9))
 (segment (start 74.78032 71.12272) (end 86.1568 82.4992) (width 0.25) (layer "B.Cu") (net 9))
 (segment (start 113.2332 76.6064) (end 116.8388 73.0008) (width 0.25) (layer "B.Cu") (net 9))
 (segment (start 72.3954 71.12272) (end 74.78032 71.12272) (width 0.25) (layer "B.Cu") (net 9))
 (segment (start 113.2332 81.4324) (end 113.2332 76.6064) (width 0.25) (layer "B.Cu") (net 9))
 (segment (start 112.8776 99.1108) (end 134.8486 99.1108) (width 0.25) (layer "F.Cu") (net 34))
 (segment (start 112.8268 99.06) (end 112.8776 99.1108) (width 0.25) (layer "F.Cu") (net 34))
 (segment (start 98.5774 88.0618) (end 101.0666 88.0618) (width 0.25) (layer "F.Cu") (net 34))
 (segment (start 101.0666 88.0618) (end 101.219 88.2142) (width 0.25) (layer "F.Cu") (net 34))
 (via (at 101.219 88.2142) (size 0.8) (drill 0.4) (layers "F.Cu" "B.Cu") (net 34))
 (via (at 98.5774 88.0618) (size 0.8) (drill 0.4) (layers "F.Cu" "B.Cu") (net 34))
 (via (at 112.8268 99.06) (size 0.8) (drill 0.4) (layers "F.Cu" "B.Cu") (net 34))
 (segment (start 112.0648 99.06) (end 112.8268 99.06) (width 0.25) (layer "B.Cu") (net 34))
 (segment (start 95.23 86.36272) (end 96.87832 86.36272) (width 0.25) (layer "B.Cu") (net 34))
 (segment (start 101.219 88.2142) (end 112.0648 99.06) (width 0.25) (layer "B.Cu") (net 34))
 (segment (start 96.87832 86.36272) (end 98.5774 88.0618) (width 0.25) (layer "B.Cu") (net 34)))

